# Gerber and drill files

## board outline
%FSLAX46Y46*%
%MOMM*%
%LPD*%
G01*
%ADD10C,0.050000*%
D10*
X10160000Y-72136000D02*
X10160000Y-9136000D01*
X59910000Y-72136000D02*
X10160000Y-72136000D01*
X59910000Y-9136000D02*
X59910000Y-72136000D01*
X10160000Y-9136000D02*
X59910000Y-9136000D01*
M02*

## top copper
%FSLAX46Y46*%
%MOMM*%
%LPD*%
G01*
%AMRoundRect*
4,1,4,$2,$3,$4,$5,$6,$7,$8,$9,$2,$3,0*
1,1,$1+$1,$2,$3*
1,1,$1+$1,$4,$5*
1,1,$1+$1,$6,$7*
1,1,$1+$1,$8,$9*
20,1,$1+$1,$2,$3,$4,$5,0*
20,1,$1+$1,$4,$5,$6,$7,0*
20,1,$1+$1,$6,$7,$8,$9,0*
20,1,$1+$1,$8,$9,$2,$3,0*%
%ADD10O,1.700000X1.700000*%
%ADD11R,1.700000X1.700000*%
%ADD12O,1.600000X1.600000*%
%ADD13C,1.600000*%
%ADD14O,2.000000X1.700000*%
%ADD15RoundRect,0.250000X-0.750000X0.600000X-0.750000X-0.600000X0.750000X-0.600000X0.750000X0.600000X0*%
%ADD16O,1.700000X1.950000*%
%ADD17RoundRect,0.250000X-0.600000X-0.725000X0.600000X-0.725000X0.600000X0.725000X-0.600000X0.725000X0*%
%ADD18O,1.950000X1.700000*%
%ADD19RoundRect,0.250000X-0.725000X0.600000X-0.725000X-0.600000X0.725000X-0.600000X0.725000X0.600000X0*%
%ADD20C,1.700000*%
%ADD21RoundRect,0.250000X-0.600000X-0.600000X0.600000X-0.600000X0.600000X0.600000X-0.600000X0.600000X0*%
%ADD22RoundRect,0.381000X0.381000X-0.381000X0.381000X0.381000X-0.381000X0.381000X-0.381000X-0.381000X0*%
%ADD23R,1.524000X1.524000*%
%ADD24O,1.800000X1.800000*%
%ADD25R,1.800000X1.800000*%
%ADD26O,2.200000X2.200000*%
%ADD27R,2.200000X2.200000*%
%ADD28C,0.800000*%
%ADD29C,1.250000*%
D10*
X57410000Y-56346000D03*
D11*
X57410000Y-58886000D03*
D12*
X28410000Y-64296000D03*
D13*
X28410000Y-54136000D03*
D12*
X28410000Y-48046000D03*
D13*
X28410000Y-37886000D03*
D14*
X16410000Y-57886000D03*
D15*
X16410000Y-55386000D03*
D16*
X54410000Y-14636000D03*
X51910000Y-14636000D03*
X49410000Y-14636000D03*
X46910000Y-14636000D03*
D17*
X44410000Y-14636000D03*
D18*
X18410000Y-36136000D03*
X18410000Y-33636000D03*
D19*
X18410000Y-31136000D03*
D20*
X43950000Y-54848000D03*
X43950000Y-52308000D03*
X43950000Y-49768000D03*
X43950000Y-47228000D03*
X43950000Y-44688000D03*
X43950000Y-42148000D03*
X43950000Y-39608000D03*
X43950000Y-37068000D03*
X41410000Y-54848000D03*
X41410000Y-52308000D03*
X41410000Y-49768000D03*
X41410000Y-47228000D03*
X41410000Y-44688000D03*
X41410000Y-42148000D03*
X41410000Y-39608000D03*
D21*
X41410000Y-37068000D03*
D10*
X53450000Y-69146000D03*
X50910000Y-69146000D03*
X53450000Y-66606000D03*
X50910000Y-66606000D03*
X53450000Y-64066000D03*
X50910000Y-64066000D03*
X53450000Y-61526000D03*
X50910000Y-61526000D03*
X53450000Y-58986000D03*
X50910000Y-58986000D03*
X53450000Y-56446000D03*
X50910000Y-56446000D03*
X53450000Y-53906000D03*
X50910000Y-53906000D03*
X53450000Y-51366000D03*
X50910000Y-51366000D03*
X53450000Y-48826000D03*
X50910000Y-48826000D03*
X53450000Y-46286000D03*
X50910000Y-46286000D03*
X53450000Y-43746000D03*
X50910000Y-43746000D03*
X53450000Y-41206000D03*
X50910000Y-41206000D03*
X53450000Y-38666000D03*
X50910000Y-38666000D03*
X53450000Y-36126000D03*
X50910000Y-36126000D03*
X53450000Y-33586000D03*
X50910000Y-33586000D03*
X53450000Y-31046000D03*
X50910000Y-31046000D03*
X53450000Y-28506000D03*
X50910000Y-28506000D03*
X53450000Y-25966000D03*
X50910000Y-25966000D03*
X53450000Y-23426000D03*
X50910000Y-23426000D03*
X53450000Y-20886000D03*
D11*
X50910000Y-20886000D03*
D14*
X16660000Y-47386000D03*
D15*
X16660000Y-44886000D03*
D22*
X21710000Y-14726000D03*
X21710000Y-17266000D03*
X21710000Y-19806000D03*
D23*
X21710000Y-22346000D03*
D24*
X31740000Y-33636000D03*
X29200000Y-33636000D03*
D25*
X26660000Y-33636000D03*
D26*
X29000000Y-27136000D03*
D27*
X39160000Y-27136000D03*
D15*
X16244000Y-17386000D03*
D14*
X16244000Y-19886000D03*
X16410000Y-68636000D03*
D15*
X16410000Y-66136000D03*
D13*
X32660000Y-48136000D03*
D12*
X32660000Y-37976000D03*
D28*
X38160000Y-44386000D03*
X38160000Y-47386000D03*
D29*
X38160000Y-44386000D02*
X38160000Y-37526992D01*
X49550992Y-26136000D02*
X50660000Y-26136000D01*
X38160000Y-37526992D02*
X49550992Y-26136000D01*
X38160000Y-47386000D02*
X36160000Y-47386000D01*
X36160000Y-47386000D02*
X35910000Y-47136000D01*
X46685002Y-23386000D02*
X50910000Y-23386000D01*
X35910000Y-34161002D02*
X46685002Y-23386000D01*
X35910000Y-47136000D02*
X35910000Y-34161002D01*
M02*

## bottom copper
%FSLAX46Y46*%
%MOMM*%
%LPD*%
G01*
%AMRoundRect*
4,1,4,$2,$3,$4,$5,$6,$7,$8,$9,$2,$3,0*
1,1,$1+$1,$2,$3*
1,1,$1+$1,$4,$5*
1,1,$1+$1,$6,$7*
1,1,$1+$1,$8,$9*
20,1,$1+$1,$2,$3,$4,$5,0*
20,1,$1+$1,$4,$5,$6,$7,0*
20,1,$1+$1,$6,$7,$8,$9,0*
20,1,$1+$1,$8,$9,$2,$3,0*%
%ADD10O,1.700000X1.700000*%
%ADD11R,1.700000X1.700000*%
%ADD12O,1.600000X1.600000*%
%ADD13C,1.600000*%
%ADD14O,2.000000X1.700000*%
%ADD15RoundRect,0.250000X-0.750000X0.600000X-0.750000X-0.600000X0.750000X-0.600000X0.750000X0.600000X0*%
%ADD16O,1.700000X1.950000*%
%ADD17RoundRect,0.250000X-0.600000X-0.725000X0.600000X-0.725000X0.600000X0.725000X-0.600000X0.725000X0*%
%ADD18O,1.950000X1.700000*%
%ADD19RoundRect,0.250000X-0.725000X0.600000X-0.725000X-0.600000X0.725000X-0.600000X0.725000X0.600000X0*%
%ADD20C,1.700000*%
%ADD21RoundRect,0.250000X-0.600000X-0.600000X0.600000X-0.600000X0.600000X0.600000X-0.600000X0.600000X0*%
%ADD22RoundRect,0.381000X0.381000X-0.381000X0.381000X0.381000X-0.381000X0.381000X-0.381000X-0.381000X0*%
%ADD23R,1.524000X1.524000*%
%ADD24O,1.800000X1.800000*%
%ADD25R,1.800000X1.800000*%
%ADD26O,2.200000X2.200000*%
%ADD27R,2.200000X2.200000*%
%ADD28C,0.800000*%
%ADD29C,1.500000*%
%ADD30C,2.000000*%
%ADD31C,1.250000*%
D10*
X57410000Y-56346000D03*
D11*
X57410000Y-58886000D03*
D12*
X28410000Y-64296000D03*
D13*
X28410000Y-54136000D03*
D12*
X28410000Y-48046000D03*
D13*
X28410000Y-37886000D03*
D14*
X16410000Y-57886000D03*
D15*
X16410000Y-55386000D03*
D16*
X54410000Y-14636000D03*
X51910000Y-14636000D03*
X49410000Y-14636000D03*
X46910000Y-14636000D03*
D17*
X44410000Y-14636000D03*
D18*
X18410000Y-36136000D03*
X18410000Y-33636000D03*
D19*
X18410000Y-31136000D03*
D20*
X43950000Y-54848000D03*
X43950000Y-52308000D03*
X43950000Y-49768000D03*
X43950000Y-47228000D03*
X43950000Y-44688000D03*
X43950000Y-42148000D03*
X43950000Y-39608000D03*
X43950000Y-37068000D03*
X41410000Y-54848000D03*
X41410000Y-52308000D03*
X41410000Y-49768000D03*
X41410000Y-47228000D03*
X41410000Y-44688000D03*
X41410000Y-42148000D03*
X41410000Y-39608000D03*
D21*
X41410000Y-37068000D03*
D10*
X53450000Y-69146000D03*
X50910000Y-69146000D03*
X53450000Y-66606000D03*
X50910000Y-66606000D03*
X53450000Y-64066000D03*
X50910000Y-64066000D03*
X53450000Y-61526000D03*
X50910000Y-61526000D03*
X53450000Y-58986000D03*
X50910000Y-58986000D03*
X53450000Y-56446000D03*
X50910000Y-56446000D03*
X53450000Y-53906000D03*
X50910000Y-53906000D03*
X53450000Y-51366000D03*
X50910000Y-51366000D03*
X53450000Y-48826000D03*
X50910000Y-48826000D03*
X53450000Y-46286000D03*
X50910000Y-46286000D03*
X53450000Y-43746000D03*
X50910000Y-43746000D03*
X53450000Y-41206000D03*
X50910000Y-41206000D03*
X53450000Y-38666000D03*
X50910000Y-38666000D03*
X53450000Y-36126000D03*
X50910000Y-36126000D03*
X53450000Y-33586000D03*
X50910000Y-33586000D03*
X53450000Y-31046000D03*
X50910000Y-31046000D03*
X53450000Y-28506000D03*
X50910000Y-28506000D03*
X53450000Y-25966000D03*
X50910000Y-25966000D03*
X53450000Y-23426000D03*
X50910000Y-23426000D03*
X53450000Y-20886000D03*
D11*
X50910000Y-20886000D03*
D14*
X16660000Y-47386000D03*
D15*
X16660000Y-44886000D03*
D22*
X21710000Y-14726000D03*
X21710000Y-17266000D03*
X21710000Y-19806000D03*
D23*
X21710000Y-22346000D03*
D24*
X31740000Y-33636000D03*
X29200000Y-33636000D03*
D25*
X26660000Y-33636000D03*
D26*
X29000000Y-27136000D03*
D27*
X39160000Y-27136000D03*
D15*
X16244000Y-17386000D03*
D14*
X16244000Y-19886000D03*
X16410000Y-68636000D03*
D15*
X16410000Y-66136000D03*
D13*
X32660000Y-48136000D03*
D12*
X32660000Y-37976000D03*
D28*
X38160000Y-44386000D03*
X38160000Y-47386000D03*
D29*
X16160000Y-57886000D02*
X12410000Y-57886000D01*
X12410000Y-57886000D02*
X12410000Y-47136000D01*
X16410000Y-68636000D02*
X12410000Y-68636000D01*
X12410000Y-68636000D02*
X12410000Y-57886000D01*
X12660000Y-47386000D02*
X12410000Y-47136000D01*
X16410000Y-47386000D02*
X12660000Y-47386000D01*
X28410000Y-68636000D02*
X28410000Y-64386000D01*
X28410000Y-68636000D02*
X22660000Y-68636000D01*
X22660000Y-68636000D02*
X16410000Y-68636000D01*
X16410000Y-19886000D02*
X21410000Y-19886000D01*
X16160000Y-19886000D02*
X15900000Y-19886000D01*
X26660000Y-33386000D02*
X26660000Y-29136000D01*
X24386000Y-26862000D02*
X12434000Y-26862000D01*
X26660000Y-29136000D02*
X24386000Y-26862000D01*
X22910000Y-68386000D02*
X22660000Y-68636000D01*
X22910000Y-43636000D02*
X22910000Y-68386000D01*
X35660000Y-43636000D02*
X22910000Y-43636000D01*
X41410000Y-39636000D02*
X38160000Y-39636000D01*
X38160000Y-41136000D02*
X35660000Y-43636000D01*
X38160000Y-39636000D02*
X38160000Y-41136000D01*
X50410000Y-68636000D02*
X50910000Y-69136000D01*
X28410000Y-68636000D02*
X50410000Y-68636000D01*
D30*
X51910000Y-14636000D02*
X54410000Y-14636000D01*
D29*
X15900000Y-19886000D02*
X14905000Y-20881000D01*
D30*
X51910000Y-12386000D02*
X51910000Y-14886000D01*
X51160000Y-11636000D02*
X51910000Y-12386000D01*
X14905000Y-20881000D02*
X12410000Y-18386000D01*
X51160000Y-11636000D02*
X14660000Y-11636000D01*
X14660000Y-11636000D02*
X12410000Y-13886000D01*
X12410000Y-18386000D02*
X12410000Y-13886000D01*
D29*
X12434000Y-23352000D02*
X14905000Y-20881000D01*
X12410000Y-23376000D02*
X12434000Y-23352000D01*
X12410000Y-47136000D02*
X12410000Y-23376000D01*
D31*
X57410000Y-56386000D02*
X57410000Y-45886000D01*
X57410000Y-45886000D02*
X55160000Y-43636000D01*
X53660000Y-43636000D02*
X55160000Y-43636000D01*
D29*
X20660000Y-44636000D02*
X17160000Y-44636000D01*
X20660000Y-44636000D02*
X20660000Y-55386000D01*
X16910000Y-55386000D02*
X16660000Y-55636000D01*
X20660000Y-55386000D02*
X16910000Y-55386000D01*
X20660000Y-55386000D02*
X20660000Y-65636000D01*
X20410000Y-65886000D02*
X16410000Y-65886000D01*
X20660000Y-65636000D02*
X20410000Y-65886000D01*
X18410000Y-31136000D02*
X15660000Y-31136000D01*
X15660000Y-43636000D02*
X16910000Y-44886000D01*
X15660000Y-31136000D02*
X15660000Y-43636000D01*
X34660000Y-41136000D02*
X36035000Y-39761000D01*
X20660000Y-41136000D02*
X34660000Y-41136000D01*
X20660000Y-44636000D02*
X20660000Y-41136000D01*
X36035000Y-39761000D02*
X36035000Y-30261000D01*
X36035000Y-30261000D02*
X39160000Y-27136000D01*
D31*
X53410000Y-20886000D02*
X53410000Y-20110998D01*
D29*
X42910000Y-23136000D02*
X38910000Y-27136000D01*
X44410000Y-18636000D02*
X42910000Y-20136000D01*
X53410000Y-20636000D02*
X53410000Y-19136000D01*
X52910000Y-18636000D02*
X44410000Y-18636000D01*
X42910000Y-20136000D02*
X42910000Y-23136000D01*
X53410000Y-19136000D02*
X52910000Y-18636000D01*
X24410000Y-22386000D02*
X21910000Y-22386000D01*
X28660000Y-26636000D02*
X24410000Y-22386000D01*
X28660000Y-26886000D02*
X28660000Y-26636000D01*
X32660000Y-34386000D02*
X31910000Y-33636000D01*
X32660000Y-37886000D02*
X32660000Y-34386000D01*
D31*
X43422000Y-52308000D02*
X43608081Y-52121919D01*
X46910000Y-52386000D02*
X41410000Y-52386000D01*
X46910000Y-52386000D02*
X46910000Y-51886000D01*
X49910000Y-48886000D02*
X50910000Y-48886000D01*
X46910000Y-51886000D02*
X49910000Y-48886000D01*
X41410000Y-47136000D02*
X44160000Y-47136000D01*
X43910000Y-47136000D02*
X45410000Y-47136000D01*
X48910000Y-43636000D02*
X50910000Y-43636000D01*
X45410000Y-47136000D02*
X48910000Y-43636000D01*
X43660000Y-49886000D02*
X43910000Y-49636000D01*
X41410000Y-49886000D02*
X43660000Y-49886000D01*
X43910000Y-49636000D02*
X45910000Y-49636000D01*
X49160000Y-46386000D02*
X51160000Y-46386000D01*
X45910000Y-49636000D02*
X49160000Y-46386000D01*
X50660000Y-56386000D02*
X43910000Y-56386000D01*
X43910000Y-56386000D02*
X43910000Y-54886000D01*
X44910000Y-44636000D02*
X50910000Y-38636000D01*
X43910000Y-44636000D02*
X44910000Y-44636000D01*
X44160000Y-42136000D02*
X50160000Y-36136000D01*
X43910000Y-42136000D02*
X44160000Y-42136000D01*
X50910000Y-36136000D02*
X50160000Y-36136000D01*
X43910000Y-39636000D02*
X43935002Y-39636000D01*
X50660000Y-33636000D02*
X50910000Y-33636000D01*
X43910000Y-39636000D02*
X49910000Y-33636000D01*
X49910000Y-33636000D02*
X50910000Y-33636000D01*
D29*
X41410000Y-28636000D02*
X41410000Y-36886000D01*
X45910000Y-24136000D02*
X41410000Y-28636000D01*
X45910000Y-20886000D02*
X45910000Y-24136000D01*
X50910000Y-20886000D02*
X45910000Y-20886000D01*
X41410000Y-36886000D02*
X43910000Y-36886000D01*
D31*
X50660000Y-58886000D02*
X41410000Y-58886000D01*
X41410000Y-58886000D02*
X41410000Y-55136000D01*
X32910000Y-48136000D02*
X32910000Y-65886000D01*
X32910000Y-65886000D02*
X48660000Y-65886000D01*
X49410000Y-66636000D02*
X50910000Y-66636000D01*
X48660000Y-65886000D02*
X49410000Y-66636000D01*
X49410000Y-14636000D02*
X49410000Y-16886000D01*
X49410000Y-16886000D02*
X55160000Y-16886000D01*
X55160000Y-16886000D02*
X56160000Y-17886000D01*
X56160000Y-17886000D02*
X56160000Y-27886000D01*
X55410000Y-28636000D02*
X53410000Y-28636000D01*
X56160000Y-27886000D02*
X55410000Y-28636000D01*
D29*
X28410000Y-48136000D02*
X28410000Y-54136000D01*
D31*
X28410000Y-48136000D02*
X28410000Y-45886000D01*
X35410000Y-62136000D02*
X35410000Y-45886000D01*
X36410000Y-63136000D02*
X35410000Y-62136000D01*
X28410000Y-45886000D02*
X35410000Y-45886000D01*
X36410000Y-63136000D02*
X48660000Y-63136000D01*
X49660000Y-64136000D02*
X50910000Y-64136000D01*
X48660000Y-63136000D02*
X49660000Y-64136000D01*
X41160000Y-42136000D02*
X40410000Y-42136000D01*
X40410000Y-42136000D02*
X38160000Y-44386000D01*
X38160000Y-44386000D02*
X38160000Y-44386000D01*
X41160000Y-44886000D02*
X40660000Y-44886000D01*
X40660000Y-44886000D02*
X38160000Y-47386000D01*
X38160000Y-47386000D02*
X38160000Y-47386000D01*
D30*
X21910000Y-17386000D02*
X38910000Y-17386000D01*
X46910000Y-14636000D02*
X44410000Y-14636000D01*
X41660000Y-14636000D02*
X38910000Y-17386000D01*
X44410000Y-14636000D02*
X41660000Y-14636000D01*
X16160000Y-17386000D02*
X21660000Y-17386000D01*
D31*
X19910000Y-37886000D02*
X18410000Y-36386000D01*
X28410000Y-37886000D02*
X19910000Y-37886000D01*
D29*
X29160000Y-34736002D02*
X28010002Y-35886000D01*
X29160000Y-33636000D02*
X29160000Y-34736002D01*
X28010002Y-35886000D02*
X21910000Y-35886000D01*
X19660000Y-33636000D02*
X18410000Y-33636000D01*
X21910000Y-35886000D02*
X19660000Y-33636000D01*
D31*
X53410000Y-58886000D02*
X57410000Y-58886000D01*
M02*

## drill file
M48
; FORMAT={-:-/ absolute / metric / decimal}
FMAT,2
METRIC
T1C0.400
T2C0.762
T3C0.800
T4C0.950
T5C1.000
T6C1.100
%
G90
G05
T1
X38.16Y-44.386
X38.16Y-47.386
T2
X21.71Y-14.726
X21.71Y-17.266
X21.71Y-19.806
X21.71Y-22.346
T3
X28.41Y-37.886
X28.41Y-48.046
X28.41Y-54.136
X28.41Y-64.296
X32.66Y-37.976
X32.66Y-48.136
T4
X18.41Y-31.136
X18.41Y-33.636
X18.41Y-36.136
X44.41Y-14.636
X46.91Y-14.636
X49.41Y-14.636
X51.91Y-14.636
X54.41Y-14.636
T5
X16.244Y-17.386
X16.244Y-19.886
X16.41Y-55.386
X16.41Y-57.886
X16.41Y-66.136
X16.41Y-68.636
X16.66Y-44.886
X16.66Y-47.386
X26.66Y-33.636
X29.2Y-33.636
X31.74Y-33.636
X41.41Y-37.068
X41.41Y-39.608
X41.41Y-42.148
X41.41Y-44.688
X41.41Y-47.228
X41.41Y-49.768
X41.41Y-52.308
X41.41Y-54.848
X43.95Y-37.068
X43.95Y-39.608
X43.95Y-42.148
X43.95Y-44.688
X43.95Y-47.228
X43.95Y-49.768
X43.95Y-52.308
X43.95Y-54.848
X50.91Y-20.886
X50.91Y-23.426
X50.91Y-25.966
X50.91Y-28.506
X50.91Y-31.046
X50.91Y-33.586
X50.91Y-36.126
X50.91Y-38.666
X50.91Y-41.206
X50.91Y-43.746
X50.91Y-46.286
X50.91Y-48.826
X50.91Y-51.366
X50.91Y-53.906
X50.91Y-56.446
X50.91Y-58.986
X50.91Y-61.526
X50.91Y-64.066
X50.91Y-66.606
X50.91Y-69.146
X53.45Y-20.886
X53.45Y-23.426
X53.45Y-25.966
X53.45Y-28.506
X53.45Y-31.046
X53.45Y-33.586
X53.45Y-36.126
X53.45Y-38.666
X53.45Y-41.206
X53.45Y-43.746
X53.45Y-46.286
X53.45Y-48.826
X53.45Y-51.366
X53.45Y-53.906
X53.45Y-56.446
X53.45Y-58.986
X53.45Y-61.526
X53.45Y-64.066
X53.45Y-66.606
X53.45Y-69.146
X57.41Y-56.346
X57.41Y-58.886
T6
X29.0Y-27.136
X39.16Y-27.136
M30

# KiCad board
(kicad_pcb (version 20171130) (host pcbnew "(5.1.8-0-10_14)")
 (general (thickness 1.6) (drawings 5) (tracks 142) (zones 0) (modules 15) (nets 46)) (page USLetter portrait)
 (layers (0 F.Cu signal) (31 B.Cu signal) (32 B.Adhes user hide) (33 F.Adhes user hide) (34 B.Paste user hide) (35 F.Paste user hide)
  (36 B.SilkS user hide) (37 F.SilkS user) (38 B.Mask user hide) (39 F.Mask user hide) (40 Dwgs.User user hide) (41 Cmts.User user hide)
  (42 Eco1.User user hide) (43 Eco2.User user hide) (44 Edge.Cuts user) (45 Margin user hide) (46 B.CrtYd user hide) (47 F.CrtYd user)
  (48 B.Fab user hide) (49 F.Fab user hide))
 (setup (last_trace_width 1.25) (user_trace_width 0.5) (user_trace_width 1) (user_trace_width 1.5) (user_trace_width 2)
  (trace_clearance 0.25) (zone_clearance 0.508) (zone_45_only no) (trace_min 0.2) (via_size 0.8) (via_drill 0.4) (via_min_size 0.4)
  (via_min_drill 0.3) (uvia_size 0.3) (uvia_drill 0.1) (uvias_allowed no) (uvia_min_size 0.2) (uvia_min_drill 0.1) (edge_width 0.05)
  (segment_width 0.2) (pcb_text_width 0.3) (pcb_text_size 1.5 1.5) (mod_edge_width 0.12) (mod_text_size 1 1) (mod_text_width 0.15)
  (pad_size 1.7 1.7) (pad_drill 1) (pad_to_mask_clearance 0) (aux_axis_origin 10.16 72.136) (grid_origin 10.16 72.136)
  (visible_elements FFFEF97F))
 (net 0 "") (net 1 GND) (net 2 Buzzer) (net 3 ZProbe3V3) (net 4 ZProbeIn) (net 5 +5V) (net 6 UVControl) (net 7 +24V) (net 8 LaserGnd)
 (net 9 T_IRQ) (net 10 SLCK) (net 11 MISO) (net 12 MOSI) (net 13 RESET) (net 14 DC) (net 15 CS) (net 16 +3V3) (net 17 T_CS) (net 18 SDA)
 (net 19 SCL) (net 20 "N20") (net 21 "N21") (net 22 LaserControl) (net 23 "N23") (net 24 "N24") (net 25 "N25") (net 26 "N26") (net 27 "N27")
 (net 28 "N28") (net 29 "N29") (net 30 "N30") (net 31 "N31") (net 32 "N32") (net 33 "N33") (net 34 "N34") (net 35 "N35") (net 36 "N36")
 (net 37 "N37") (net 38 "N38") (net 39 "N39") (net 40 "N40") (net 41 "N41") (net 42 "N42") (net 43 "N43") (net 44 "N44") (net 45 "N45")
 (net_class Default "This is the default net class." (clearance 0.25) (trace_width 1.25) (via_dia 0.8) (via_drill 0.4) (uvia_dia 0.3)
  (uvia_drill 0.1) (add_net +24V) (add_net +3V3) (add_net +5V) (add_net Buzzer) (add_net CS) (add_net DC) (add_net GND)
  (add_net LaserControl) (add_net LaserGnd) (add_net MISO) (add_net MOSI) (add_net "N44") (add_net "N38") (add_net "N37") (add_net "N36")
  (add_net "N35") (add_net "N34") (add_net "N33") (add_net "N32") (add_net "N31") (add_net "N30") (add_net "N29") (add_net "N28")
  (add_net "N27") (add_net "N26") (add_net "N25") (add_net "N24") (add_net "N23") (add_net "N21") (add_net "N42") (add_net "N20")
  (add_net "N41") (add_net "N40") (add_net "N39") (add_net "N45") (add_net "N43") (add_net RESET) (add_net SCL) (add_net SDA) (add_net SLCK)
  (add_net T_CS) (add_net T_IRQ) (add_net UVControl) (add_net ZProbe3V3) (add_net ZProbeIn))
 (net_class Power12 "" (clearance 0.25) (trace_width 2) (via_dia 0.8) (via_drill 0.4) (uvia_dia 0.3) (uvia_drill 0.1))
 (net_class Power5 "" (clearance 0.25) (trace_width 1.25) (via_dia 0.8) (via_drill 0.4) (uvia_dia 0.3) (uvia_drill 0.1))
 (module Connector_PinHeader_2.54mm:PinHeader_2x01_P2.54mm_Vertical (layer F.Cu) (at 57.41 58.886 90)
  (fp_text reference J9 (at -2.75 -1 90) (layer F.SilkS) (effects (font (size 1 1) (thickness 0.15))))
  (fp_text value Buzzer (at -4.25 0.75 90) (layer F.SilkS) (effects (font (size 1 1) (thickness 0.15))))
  (pad 2 thru_hole oval (at 2.54 0 90) (size 1.7 1.7) (drill 1) (layers *.Cu *.Mask) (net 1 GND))
  (pad 1 thru_hole rect (at 0 0 90) (size 1.7 1.7) (drill 1) (layers *.Cu *.Mask) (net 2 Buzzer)))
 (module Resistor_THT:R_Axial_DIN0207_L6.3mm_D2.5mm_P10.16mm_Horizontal (layer F.Cu) (at 28.41 54.136 270)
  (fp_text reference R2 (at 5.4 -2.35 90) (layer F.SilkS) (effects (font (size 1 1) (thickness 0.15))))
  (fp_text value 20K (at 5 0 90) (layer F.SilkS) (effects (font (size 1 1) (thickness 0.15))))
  (pad 2 thru_hole oval (at 10.16 0 270) (size 1.6 1.6) (drill 0.8) (layers *.Cu *.Mask) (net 1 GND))
  (pad 1 thru_hole circle (at 0 0 270) (size 1.6 1.6) (drill 0.8) (layers *.Cu *.Mask) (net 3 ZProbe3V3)))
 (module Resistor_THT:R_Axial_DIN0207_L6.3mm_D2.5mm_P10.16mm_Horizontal (layer F.Cu) (at 28.41 37.886 270)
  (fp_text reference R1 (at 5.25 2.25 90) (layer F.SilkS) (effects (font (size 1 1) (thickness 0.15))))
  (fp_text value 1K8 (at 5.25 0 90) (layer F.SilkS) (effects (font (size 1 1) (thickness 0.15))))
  (pad 2 thru_hole oval (at 10.16 0 270) (size 1.6 1.6) (drill 0.8) (layers *.Cu *.Mask) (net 3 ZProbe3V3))
  (pad 1 thru_hole circle (at 0 0 270) (size 1.6 1.6) (drill 0.8) (layers *.Cu *.Mask) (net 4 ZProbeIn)))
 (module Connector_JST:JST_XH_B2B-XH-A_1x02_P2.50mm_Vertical (layer F.Cu) (at 16.41 55.386 270)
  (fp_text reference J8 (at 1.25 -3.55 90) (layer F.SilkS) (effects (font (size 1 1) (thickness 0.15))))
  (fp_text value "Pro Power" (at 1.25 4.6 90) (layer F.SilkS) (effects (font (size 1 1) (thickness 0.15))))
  (pad 2 thru_hole oval (at 2.5 0 270) (size 1.7 2) (drill 1) (layers *.Cu *.Mask) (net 1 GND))
  (pad 1 thru_hole roundrect (at 0 0 270) (size 1.7 2) (drill 1) (layers *.Cu *.Mask) (roundrect_rratio 0.1470588235294118) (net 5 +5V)))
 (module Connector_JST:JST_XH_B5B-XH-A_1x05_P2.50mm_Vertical (layer F.Cu) (at 44.41 14.636)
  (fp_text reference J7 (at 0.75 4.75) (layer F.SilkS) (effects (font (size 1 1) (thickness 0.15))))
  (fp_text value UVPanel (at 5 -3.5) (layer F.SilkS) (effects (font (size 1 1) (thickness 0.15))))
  (pad 5 thru_hole oval (at 10 0) (size 1.7 1.95) (drill 0.95) (layers *.Cu *.Mask) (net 1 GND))
  (pad 4 thru_hole oval (at 7.5 0) (size 1.7 1.95) (drill 0.95) (layers *.Cu *.Mask) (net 1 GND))
  (pad 3 thru_hole oval (at 5 0) (size 1.7 1.95) (drill 0.95) (layers *.Cu *.Mask) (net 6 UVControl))
  (pad 2 thru_hole oval (at 2.5 0) (size 1.7 1.95) (drill 0.95) (layers *.Cu *.Mask) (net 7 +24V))
  (pad 1 thru_hole roundrect (at 0 0) (size 1.7 1.95) (drill 0.95) (layers *.Cu *.Mask) (roundrect_rratio 0.1470588235294118) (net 7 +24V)))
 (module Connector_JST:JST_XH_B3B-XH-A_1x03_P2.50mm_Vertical (layer F.Cu) (at 18.41 31.136 270)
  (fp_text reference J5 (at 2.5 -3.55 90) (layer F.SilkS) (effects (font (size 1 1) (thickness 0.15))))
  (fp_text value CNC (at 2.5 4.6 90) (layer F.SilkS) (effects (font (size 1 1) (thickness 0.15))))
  (pad 3 thru_hole oval (at 5 0 270) (size 1.7 1.95) (drill 0.95) (layers *.Cu *.Mask) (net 4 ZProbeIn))
  (pad 2 thru_hole oval (at 2.5 0 270) (size 1.7 1.95) (drill 0.95) (layers *.Cu *.Mask) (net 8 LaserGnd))
  (pad 1 thru_hole roundrect (at 0 0 270) (size 1.7 1.95) (drill 0.95) (layers *.Cu *.Mask) (roundrect_rratio 0.1470588235294118)
   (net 5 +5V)))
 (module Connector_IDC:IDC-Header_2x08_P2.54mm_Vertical (layer F.Cu) (at 41.41 37.068)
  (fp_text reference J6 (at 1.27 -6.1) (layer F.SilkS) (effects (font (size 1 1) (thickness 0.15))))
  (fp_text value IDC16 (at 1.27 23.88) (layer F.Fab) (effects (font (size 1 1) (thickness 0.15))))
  (pad 16 thru_hole circle (at 2.54 17.78) (size 1.7 1.7) (drill 1) (layers *.Cu *.Mask) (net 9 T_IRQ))
  (pad 14 thru_hole circle (at 2.54 15.24) (size 1.7 1.7) (drill 1) (layers *.Cu *.Mask) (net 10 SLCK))
  (pad 12 thru_hole circle (at 2.54 12.7) (size 1.7 1.7) (drill 1) (layers *.Cu *.Mask) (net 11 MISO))
  (pad 10 thru_hole circle (at 2.54 10.16) (size 1.7 1.7) (drill 1) (layers *.Cu *.Mask) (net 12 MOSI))
  (pad 8 thru_hole circle (at 2.54 7.62) (size 1.7 1.7) (drill 1) (layers *.Cu *.Mask) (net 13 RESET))
  (pad 6 thru_hole circle (at 2.54 5.08) (size 1.7 1.7) (drill 1) (layers *.Cu *.Mask) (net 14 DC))
  (pad 4 thru_hole circle (at 2.54 2.54) (size 1.7 1.7) (drill 1) (layers *.Cu *.Mask) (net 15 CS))
  (pad 2 thru_hole circle (at 2.54 0) (size 1.7 1.7) (drill 1) (layers *.Cu *.Mask) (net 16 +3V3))
  (pad 15 thru_hole circle (at 0 17.78) (size 1.7 1.7) (drill 1) (layers *.Cu *.Mask) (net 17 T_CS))
  (pad 13 thru_hole circle (at 0 15.24) (size 1.7 1.7) (drill 1) (layers *.Cu *.Mask) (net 10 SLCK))
  (pad 11 thru_hole circle (at 0 12.7) (size 1.7 1.7) (drill 1) (layers *.Cu *.Mask) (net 11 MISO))
  (pad 9 thru_hole circle (at 0 10.16) (size 1.7 1.7) (drill 1) (layers *.Cu *.Mask) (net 12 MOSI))
  (pad 7 thru_hole circle (at 0 7.62) (size 1.7 1.7) (drill 1) (layers *.Cu *.Mask) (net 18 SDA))
  (pad 5 thru_hole circle (at 0 5.08) (size 1.7 1.7) (drill 1) (layers *.Cu *.Mask) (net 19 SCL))
  (pad 3 thru_hole circle (at 0 2.54) (size 1.7 1.7) (drill 1) (layers *.Cu *.Mask) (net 1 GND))
  (pad 1 thru_hole roundrect (at 0 0) (size 1.7 1.7) (drill 1) (layers *.Cu *.Mask) (roundrect_rratio 0.1470588235294118) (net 16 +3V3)))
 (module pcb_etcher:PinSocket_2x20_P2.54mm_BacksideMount (layer F.Cu) (at 50.91 20.886)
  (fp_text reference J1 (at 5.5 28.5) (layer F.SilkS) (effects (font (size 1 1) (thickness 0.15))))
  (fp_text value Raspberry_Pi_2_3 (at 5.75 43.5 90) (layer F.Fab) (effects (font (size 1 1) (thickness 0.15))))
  (pad 40 thru_hole oval (at 2.54 48.26) (size 1.7 1.7) (drill 1) (layers *.Cu *.Mask) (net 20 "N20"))
  (pad 39 thru_hole oval (at 0 48.26) (size 1.7 1.7) (drill 1) (layers *.Cu *.Mask) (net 1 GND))
  (pad 38 thru_hole oval (at 2.54 45.72) (size 1.7 1.7) (drill 1) (layers *.Cu *.Mask) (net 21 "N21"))
  (pad 37 thru_hole oval (at 0 45.72) (size 1.7 1.7) (drill 1) (layers *.Cu *.Mask) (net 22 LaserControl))
  (pad 36 thru_hole oval (at 2.54 43.18) (size 1.7 1.7) (drill 1) (layers *.Cu *.Mask) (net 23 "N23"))
  (pad 35 thru_hole oval (at 0 43.18) (size 1.7 1.7) (drill 1) (layers *.Cu *.Mask) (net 3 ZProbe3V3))
  (pad 34 thru_hole oval (at 2.54 40.64) (size 1.7 1.7) (drill 1) (layers *.Cu *.Mask) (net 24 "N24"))
  (pad 33 thru_hole oval (at 0 40.64) (size 1.7 1.7) (drill 1) (layers *.Cu *.Mask) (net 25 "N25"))
  (pad 32 thru_hole oval (at 2.54 38.1) (size 1.7 1.7) (drill 1) (layers *.Cu *.Mask) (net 2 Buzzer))
  (pad 31 thru_hole oval (at 0 38.1) (size 1.7 1.7) (drill 1) (layers *.Cu *.Mask) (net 17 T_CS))
  (pad 30 thru_hole oval (at 2.54 35.56) (size 1.7 1.7) (drill 1) (layers *.Cu *.Mask) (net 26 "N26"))
  (pad 29 thru_hole oval (at 0 35.56) (size 1.7 1.7) (drill 1) (layers *.Cu *.Mask) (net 9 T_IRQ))
  (pad 28 thru_hole oval (at 2.54 33.02) (size 1.7 1.7) (drill 1) (layers *.Cu *.Mask) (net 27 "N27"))
  (pad 27 thru_hole oval (at 0 33.02) (size 1.7 1.7) (drill 1) (layers *.Cu *.Mask) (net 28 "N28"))
  (pad 26 thru_hole oval (at 2.54 30.48) (size 1.7 1.7) (drill 1) (layers *.Cu *.Mask) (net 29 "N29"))
  (pad 25 thru_hole oval (at 0 30.48) (size 1.7 1.7) (drill 1) (layers *.Cu *.Mask) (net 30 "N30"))
  (pad 24 thru_hole oval (at 2.54 27.94) (size 1.7 1.7) (drill 1) (layers *.Cu *.Mask) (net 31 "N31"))
  (pad 23 thru_hole oval (at 0 27.94) (size 1.7 1.7) (drill 1) (layers *.Cu *.Mask) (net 10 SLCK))
  (pad 22 thru_hole oval (at 2.54 25.4) (size 1.7 1.7) (drill 1) (layers *.Cu *.Mask) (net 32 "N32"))
  (pad 21 thru_hole oval (at 0 25.4) (size 1.7 1.7) (drill 1) (layers *.Cu *.Mask) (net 11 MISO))
  (pad 20 thru_hole oval (at 2.54 22.86) (size 1.7 1.7) (drill 1) (layers *.Cu *.Mask) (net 1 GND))
  (pad 19 thru_hole oval (at 0 22.86) (size 1.7 1.7) (drill 1) (layers *.Cu *.Mask) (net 12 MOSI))
  (pad 18 thru_hole oval (at 2.54 20.32) (size 1.7 1.7) (drill 1) (layers *.Cu *.Mask) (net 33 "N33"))
  (pad 17 thru_hole oval (at 0 20.32) (size 1.7 1.7) (drill 1) (layers *.Cu *.Mask) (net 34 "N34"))
  (pad 16 thru_hole oval (at 2.54 17.78) (size 1.7 1.7) (drill 1) (layers *.Cu *.Mask) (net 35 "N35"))
  (pad 15 thru_hole oval (at 0 17.78) (size 1.7 1.7) (drill 1) (layers *.Cu *.Mask) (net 13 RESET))
  (pad 14 thru_hole oval (at 2.54 15.24) (size 1.7 1.7) (drill 1) (layers *.Cu *.Mask) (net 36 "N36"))
  (pad 13 thru_hole oval (at 0 15.24) (size 1.7 1.7) (drill 1) (layers *.Cu *.Mask) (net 14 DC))
  (pad 12 thru_hole oval (at 2.54 12.7) (size 1.7 1.7) (drill 1) (layers *.Cu *.Mask) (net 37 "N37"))
  (pad 11 thru_hole oval (at 0 12.7) (size 1.7 1.7) (drill 1) (layers *.Cu *.Mask) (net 15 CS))
  (pad 10 thru_hole oval (at 2.54 10.16) (size 1.7 1.7) (drill 1) (layers *.Cu *.Mask) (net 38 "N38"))
  (pad 9 thru_hole oval (at 0 10.16) (size 1.7 1.7) (drill 1) (layers *.Cu *.Mask) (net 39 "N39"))
  (pad 8 thru_hole oval (at 2.54 7.62) (size 1.7 1.7) (drill 1) (layers *.Cu *.Mask) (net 6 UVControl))
  (pad 7 thru_hole oval (at 0 7.62) (size 1.7 1.7) (drill 1) (layers *.Cu *.Mask) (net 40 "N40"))
  (pad 6 thru_hole oval (at 2.54 5.08) (size 1.7 1.7) (drill 1) (layers *.Cu *.Mask) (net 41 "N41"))
  (pad 5 thru_hole oval (at 0 5.08) (size 1.7 1.7) (drill 1) (layers *.Cu *.Mask) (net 19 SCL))
  (pad 4 thru_hole oval (at 2.54 2.54) (size 1.7 1.7) (drill 1) (layers *.Cu *.Mask) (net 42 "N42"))
  (pad 3 thru_hole oval (at 0 2.54) (size 1.7 1.7) (drill 1) (layers *.Cu *.Mask) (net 18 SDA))
  (pad 2 thru_hole oval (at 2.54 0) (size 1.7 1.7) (drill 1) (layers *.Cu *.Mask) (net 5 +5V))
  (pad 1 thru_hole rect (at 0 0) (size 1.7 1.7) (drill 1) (layers *.Cu *.Mask) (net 16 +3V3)))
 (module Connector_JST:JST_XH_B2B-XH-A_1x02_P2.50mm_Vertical (layer F.Cu) (at 16.66 44.886 270)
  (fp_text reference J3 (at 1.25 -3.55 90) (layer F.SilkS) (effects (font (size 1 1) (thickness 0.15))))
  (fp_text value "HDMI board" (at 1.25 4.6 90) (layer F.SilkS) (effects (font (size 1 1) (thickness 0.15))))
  (pad 2 thru_hole oval (at 2.5 0 270) (size 1.7 2) (drill 1) (layers *.Cu *.Mask) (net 1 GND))
  (pad 1 thru_hole roundrect (at 0 0 270) (size 1.7 2) (drill 1) (layers *.Cu *.Mask) (roundrect_rratio 0.1470588235294118) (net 5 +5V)))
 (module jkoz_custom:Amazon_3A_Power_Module (layer F.Cu) (at 29.66 18.636 90)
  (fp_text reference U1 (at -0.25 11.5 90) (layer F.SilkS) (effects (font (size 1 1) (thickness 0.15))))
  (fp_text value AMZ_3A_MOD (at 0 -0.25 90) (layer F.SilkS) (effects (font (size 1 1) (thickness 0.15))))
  (pad 4 thru_hole roundrect (at 3.91 -7.95 90) (size 1.524 1.524) (drill 0.762) (layers *.Cu *.Mask) (roundrect_rratio 0.25) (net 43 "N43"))
  (pad 3 thru_hole roundrect (at 1.37 -7.95 90) (size 1.524 1.524) (drill 0.762) (layers *.Cu *.Mask) (roundrect_rratio 0.25) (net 7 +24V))
  (pad 2 thru_hole roundrect (at -1.17 -7.95 90) (size 1.524 1.524) (drill 0.762) (layers *.Cu *.Mask) (roundrect_rratio 0.25) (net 1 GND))
  (pad 1 thru_hole rect (at -3.71 -7.95 90) (size 1.524 1.524) (drill 0.762) (layers *.Cu *.Mask) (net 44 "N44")))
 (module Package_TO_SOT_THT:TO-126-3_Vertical (layer F.Cu) (at 26.66 33.636)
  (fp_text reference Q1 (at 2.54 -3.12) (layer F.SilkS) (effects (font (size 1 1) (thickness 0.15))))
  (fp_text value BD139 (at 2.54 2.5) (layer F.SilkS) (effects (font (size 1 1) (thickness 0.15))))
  (pad 3 thru_hole oval (at 5.08 0) (size 1.8 1.8) (drill 1) (layers *.Cu *.Mask) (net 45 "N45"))
  (pad 2 thru_hole oval (at 2.54 0) (size 1.8 1.8) (drill 1) (layers *.Cu *.Mask) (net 8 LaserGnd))
  (pad 1 thru_hole rect (at 0 0) (size 1.8 1.8) (drill 1) (layers *.Cu *.Mask) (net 1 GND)))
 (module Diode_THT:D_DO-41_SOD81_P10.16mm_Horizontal (layer F.Cu) (at 39.16 27.136 180)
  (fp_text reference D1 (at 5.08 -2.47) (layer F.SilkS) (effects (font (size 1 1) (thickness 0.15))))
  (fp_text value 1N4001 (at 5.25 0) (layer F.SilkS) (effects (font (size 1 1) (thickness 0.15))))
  (pad 2 thru_hole oval (at 10.16 0 180) (size 2.2 2.2) (drill 1.1) (layers *.Cu *.Mask) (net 44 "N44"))
  (pad 1 thru_hole rect (at 0 0 180) (size 2.2 2.2) (drill 1.1) (layers *.Cu *.Mask) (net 5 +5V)))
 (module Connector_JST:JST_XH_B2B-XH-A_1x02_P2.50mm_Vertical (layer F.Cu) (at 16.244 17.386 270)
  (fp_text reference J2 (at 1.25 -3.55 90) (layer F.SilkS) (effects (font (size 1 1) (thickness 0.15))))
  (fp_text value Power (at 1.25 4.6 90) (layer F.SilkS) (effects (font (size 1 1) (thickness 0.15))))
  (pad 1 thru_hole roundrect (at 0 0 270) (size 1.7 2) (drill 1) (layers *.Cu *.Mask) (roundrect_rratio 0.1470588235294118) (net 7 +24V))
  (pad 2 thru_hole oval (at 2.5 0 270) (size 1.7 2) (drill 1) (layers *.Cu *.Mask) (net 1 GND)))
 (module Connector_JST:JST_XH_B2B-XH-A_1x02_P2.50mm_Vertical (layer F.Cu) (at 16.41 66.136 270)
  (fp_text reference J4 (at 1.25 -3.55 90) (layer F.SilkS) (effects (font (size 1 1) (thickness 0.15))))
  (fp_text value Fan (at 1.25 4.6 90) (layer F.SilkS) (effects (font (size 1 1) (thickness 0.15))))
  (pad 2 thru_hole oval (at 2.5 0 270) (size 1.7 2) (drill 1) (layers *.Cu *.Mask) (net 1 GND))
  (pad 1 thru_hole roundrect (at 0 0 270) (size 1.7 2) (drill 1) (layers *.Cu *.Mask) (roundrect_rratio 0.1470588235294118) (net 5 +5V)))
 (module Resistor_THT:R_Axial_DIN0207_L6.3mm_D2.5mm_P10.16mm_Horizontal (layer F.Cu) (at 32.66 48.136 90)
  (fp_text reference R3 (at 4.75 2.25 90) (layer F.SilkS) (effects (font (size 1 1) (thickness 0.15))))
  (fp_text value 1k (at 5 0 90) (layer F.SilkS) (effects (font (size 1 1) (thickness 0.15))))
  (pad 1 thru_hole circle (at 0 0 90) (size 1.6 1.6) (drill 0.8) (layers *.Cu *.Mask) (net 22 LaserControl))
  (pad 2 thru_hole oval (at 10.16 0 90) (size 1.6 1.6) (drill 0.8) (layers *.Cu *.Mask) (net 45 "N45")))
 (gr_line (start 10.16 72.136) (end 10.16 9.136) (layer Edge.Cuts) (width 0.05))
 (gr_line (start 59.91 72.136) (end 10.16 72.136) (layer Edge.Cuts) (width 0.05))
 (gr_line (start 59.91 9.136) (end 59.91 72.136) (layer Edge.Cuts) (width 0.05))
 (gr_line (start 10.16 9.136) (end 59.91 9.136) (layer Edge.Cuts) (width 0.05))
 (segment (start 16.16 57.886) (end 12.41 57.886) (width 1.5) (layer B.Cu) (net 1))
 (segment (start 12.41 57.886) (end 12.41 47.136) (width 1.5) (layer B.Cu) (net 1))
 (segment (start 16.41 68.636) (end 12.41 68.636) (width 1.5) (layer B.Cu) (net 1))
 (segment (start 12.41 68.636) (end 12.41 57.886) (width 1.5) (layer B.Cu) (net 1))
 (segment (start 12.66 47.386) (end 12.41 47.136) (width 1.5) (layer B.Cu) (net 1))
 (segment (start 16.41 47.386) (end 12.66 47.386) (width 1.5) (layer B.Cu) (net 1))
 (segment (start 28.41 68.636) (end 28.41 64.386) (width 1.5) (layer B.Cu) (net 1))
 (segment (start 28.41 68.636) (end 22.66 68.636) (width 1.5) (layer B.Cu) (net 1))
 (segment (start 22.66 68.636) (end 16.41 68.636) (width 1.5) (layer B.Cu) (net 1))
 (segment (start 16.41 19.886) (end 21.41 19.886) (width 1.5) (layer B.Cu) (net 1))
 (segment (start 16.16 19.886) (end 15.9 19.886) (width 1.5) (layer B.Cu) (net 1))
 (segment (start 26.66 33.386) (end 26.66 29.136) (width 1.5) (layer B.Cu) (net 1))
 (segment (start 24.386 26.862) (end 12.434 26.862) (width 1.5) (layer B.Cu) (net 1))
 (segment (start 26.66 29.136) (end 24.386 26.862) (width 1.5) (layer B.Cu) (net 1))
 (segment (start 22.91 68.386) (end 22.66 68.636) (width 1.5) (layer B.Cu) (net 1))
 (segment (start 22.91 43.636) (end 22.91 68.386) (width 1.5) (layer B.Cu) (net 1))
 (segment (start 35.66 43.636) (end 22.91 43.636) (width 1.5) (layer B.Cu) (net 1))
 (segment (start 41.41 39.636) (end 38.16 39.636) (width 1.5) (layer B.Cu) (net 1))
 (segment (start 38.16 41.136) (end 35.66 43.636) (width 1.5) (layer B.Cu) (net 1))
 (segment (start 38.16 39.636) (end 38.16 41.136) (width 1.5) (layer B.Cu) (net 1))
 (segment (start 50.41 68.636) (end 50.91 69.136) (width 1.5) (layer B.Cu) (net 1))
 (segment (start 28.41 68.636) (end 50.41 68.636) (width 1.5) (layer B.Cu) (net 1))
 (segment (start 51.91 14.636) (end 54.41 14.636) (width 2) (layer B.Cu) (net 1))
 (segment (start 15.9 19.886) (end 14.905 20.881) (width 1.5) (layer B.Cu) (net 1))
 (segment (start 51.91 12.386) (end 51.91 14.886) (width 2) (layer B.Cu) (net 1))
 (segment (start 51.16 11.636) (end 51.91 12.386) (width 2) (layer B.Cu) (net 1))
 (segment (start 14.905 20.881) (end 12.41 18.386) (width 2) (layer B.Cu) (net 1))
 (segment (start 51.16 11.636) (end 14.66 11.636) (width 2) (layer B.Cu) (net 1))
 (segment (start 14.66 11.636) (end 12.41 13.886) (width 2) (layer B.Cu) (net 1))
 (segment (start 12.41 18.386) (end 12.41 13.886) (width 2) (layer B.Cu) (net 1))
 (segment (start 12.434 23.352) (end 14.905 20.881) (width 1.5) (layer B.Cu) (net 1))
 (segment (start 12.41 23.376) (end 12.434 23.352) (width 1.5) (layer B.Cu) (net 1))
 (segment (start 12.41 47.136) (end 12.41 23.376) (width 1.5) (layer B.Cu) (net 1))
 (segment (start 57.41 56.386) (end 57.41 45.886) (width 1.25) (layer B.Cu) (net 1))
 (segment (start 57.41 45.886) (end 55.16 43.636) (width 1.25) (layer B.Cu) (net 1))
 (segment (start 53.66 43.636) (end 55.16 43.636) (width 1.25) (layer B.Cu) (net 1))
 (segment (start 20.66 44.636) (end 17.16 44.636) (width 1.5) (layer B.Cu) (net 5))
 (segment (start 20.66 44.636) (end 20.66 55.386) (width 1.5) (layer B.Cu) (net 5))
 (segment (start 16.91 55.386) (end 16.66 55.636) (width 1.5) (layer B.Cu) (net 5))
 (segment (start 20.66 55.386) (end 16.91 55.386) (width 1.5) (layer B.Cu) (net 5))
 (segment (start 20.66 55.386) (end 20.66 65.636) (width 1.5) (layer B.Cu) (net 5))
 (segment (start 20.41 65.886) (end 16.41 65.886) (width 1.5) (layer B.Cu) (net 5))
 (segment (start 20.66 65.636) (end 20.41 65.886) (width 1.5) (layer B.Cu) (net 5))
 (segment (start 18.41 31.136) (end 15.66 31.136) (width 1.5) (layer B.Cu) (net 5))
 (segment (start 15.66 43.636) (end 16.91 44.886) (width 1.5) (layer B.Cu) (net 5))
 (segment (start 15.66 31.136) (end 15.66 43.636) (width 1.5) (layer B.Cu) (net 5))
 (segment (start 34.66 41.136) (end 36.035 39.761) (width 1.5) (layer B.Cu) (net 5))
 (segment (start 20.66 41.136) (end 34.66 41.136) (width 1.5) (layer B.Cu) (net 5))
 (segment (start 20.66 44.636) (end 20.66 41.136) (width 1.5) (layer B.Cu) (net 5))
 (segment (start 36.035 39.761) (end 36.035 30.261) (width 1.5) (layer B.Cu) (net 5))
 (segment (start 36.035 30.261) (end 39.16 27.136) (width 1.5) (layer B.Cu) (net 5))
 (segment (start 53.41 20.886) (end 53.41 20.110998) (width 1.25) (layer B.Cu) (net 5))
 (segment (start 42.91 23.136) (end 38.91 27.136) (width 1.5) (layer B.Cu) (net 5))
 (segment (start 44.41 18.636) (end 42.91 20.136) (width 1.5) (layer B.Cu) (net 5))
 (segment (start 53.41 20.636) (end 53.41 19.136) (width 1.5) (layer B.Cu) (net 5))
 (segment (start 52.91 18.636) (end 44.41 18.636) (width 1.5) (layer B.Cu) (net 5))
 (segment (start 42.91 20.136) (end 42.91 23.136) (width 1.5) (layer B.Cu) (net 5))
 (segment (start 53.41 19.136) (end 52.91 18.636) (width 1.5) (layer B.Cu) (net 5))
 (segment (start 24.41 22.386) (end 21.91 22.386) (width 1.5) (layer B.Cu) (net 44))
 (segment (start 28.66 26.636) (end 24.41 22.386) (width 1.5) (layer B.Cu) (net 44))
 (segment (start 28.66 26.886) (end 28.66 26.636) (width 1.5) (layer B.Cu) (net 44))
 (segment (start 32.66 34.386) (end 31.91 33.636) (width 1.5) (layer B.Cu) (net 45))
 (segment (start 32.66 37.886) (end 32.66 34.386) (width 1.5) (layer B.Cu) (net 45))
 (segment (start 43.422 52.308) (end 43.608081 52.121919) (width 1.25) (layer B.Cu) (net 10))
 (segment (start 46.91 52.386) (end 41.41 52.386) (width 1.25) (layer B.Cu) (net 10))
 (segment (start 46.91 52.386) (end 46.91 51.886) (width 1.25) (layer B.Cu) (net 10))
 (segment (start 49.91 48.886) (end 50.91 48.886) (width 1.25) (layer B.Cu) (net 10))
 (segment (start 46.91 51.886) (end 49.91 48.886) (width 1.25) (layer B.Cu) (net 10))
 (segment (start 41.41 47.136) (end 44.16 47.136) (width 1.25) (layer B.Cu) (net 12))
 (segment (start 43.91 47.136) (end 45.41 47.136) (width 1.25) (layer B.Cu) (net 12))
 (segment (start 48.91 43.636) (end 50.91 43.636) (width 1.25) (layer B.Cu) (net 12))
 (segment (start 45.41 47.136) (end 48.91 43.636) (width 1.25) (layer B.Cu) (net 12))
 (segment (start 43.66 49.886) (end 43.91 49.636) (width 1.25) (layer B.Cu) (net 11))
 (segment (start 41.41 49.886) (end 43.66 49.886) (width 1.25) (layer B.Cu) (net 11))
 (segment (start 43.91 49.636) (end 45.91 49.636) (width 1.25) (layer B.Cu) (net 11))
 (segment (start 49.16 46.386) (end 51.16 46.386) (width 1.25) (layer B.Cu) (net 11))
 (segment (start 45.91 49.636) (end 49.16 46.386) (width 1.25) (layer B.Cu) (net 11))
 (segment (start 50.66 56.386) (end 43.91 56.386) (width 1.25) (layer B.Cu) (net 9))
 (segment (start 43.91 56.386) (end 43.91 54.886) (width 1.25) (layer B.Cu) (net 9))
 (segment (start 44.91 44.636) (end 50.91 38.636) (width 1.25) (layer B.Cu) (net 13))
 (segment (start 43.91 44.636) (end 44.91 44.636) (width 1.25) (layer B.Cu) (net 13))
 (segment (start 44.16 42.136) (end 50.16 36.136) (width 1.25) (layer B.Cu) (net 14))
 (segment (start 43.91 42.136) (end 44.16 42.136) (width 1.25) (layer B.Cu) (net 14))
 (segment (start 50.91 36.136) (end 50.16 36.136) (width 1.25) (layer B.Cu) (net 14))
 (segment (start 43.91 39.636) (end 43.935002 39.636) (width 1.25) (layer B.Cu) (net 15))
 (segment (start 50.66 33.636) (end 50.91 33.636) (width 1.25) (layer B.Cu) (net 15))
 (segment (start 43.91 39.636) (end 49.91 33.636) (width 1.25) (layer B.Cu) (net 15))
 (segment (start 49.91 33.636) (end 50.91 33.636) (width 1.25) (layer B.Cu) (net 15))
 (segment (start 41.41 28.636) (end 41.41 36.886) (width 1.5) (layer B.Cu) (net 16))
 (segment (start 45.91 24.136) (end 41.41 28.636) (width 1.5) (layer B.Cu) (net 16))
 (segment (start 45.91 20.886) (end 45.91 24.136) (width 1.5) (layer B.Cu) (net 16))
 (segment (start 50.91 20.886) (end 45.91 20.886) (width 1.5) (layer B.Cu) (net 16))
 (segment (start 41.41 36.886) (end 43.91 36.886) (width 1.5) (layer B.Cu) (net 16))
 (segment (start 50.66 58.886) (end 41.41 58.886) (width 1.25) (layer B.Cu) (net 17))
 (segment (start 41.41 58.886) (end 41.41 55.136) (width 1.25) (layer B.Cu) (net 17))
 (segment (start 32.91 48.136) (end 32.91 65.886) (width 1.25) (layer B.Cu) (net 22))
 (segment (start 32.91 65.886) (end 48.66 65.886) (width 1.25) (layer B.Cu) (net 22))
 (segment (start 49.41 66.636) (end 50.91 66.636) (width 1.25) (layer B.Cu) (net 22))
 (segment (start 48.66 65.886) (end 49.41 66.636) (width 1.25) (layer B.Cu) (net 22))
 (segment (start 49.41 14.636) (end 49.41 16.886) (width 1.25) (layer B.Cu) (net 6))
 (segment (start 49.41 16.886) (end 55.16 16.886) (width 1.25) (layer B.Cu) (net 6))
 (segment (start 55.16 16.886) (end 56.16 17.886) (width 1.25) (layer B.Cu) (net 6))
 (segment (start 56.16 17.886) (end 56.16 27.886) (width 1.25) (layer B.Cu) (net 6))
 (segment (start 55.41 28.636) (end 53.41 28.636) (width 1.25) (layer B.Cu) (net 6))
 (segment (start 56.16 27.886) (end 55.41 28.636) (width 1.25) (layer B.Cu) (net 6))
 (segment (start 28.41 48.136) (end 28.41 54.136) (width 1.5) (layer B.Cu) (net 3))
 (segment (start 28.41 48.136) (end 28.41 45.886) (width 1.25) (layer B.Cu) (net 3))
 (segment (start 35.41 62.136) (end 35.41 45.886) (width 1.25) (layer B.Cu) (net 3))
 (segment (start 36.41 63.136) (end 35.41 62.136) (width 1.25) (layer B.Cu) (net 3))
 (segment (start 28.41 45.886) (end 35.41 45.886) (width 1.25) (layer B.Cu) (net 3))
 (segment (start 36.41 63.136) (end 48.66 63.136) (width 1.25) (layer B.Cu) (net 3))
 (segment (start 49.66 64.136) (end 50.91 64.136) (width 1.25) (layer B.Cu) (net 3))
 (segment (start 48.66 63.136) (end 49.66 64.136) (width 1.25) (layer B.Cu) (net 3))
 (segment (start 41.16 42.136) (end 40.41 42.136) (width 1.25) (layer B.Cu) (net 19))
 (segment (start 40.41 42.136) (end 38.16 44.386) (width 1.25) (layer B.Cu) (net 19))
 (segment (start 38.16 44.386) (end 38.16 44.386) (width 1.25) (layer B.Cu) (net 19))
 (via (at 38.16 44.386) (size 0.8) (drill 0.4) (layers F.Cu B.Cu) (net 19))
 (segment (start 38.16 44.386) (end 38.16 37.526992) (width 1.25) (layer F.Cu) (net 19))
 (segment (start 49.550992 26.136) (end 50.66 26.136) (width 1.25) (layer F.Cu) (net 19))
 (segment (start 38.16 37.526992) (end 49.550992 26.136) (width 1.25) (layer F.Cu) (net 19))
 (segment (start 41.16 44.886) (end 40.66 44.886) (width 1.25) (layer B.Cu) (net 18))
 (segment (start 40.66 44.886) (end 38.16 47.386) (width 1.25) (layer B.Cu) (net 18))
 (segment (start 38.16 47.386) (end 38.16 47.386) (width 1.25) (layer B.Cu) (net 18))
 (via (at 38.16 47.386) (size 0.8) (drill 0.4) (layers F.Cu B.Cu) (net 18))
 (segment (start 38.16 47.386) (end 36.16 47.386) (width 1.25) (layer F.Cu) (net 18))
 (segment (start 36.16 47.386) (end 35.91 47.136) (width 1.25) (layer F.Cu) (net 18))
 (segment (start 46.685002 23.386) (end 50.91 23.386) (width 1.25) (layer F.Cu) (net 18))
 (segment (start 35.91 34.161002) (end 46.685002 23.386) (width 1.25) (layer F.Cu) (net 18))
 (segment (start 35.91 47.136) (end 35.91 34.161002) (width 1.25) (layer F.Cu) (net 18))
 (segment (start 21.91 17.386) (end 38.91 17.386) (width 2) (layer B.Cu) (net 7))
 (segment (start 46.91 14.636) (end 44.41 14.636) (width 2) (layer B.Cu) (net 7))
 (segment (start 41.66 14.636) (end 38.91 17.386) (width 2) (layer B.Cu) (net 7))
 (segment (start 44.41 14.636) (end 41.66 14.636) (width 2) (layer B.Cu) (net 7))
 (segment (start 16.16 17.386) (end 21.66 17.386) (width 2) (layer B.Cu) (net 7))
 (segment (start 19.91 37.886) (end 18.41 36.386) (width 1.25) (layer B.Cu) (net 4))
 (segment (start 28.41 37.886) (end 19.91 37.886) (width 1.25) (layer B.Cu) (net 4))
 (segment (start 29.16 34.736002) (end 28.010002 35.886) (width 1.5) (layer B.Cu) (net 8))
 (segment (start 29.16 33.636) (end 29.16 34.736002) (width 1.5) (layer B.Cu) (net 8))
 (segment (start 28.010002 35.886) (end 21.91 35.886) (width 1.5) (layer B.Cu) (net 8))
 (segment (start 19.66 33.636) (end 18.41 33.636) (width 1.5) (layer B.Cu) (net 8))
 (segment (start 21.91 35.886) (end 19.66 33.636) (width 1.5) (layer B.Cu) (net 8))
 (segment (start 53.41 58.886) (end 57.41 58.886) (width 1.25) (layer B.Cu) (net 2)))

